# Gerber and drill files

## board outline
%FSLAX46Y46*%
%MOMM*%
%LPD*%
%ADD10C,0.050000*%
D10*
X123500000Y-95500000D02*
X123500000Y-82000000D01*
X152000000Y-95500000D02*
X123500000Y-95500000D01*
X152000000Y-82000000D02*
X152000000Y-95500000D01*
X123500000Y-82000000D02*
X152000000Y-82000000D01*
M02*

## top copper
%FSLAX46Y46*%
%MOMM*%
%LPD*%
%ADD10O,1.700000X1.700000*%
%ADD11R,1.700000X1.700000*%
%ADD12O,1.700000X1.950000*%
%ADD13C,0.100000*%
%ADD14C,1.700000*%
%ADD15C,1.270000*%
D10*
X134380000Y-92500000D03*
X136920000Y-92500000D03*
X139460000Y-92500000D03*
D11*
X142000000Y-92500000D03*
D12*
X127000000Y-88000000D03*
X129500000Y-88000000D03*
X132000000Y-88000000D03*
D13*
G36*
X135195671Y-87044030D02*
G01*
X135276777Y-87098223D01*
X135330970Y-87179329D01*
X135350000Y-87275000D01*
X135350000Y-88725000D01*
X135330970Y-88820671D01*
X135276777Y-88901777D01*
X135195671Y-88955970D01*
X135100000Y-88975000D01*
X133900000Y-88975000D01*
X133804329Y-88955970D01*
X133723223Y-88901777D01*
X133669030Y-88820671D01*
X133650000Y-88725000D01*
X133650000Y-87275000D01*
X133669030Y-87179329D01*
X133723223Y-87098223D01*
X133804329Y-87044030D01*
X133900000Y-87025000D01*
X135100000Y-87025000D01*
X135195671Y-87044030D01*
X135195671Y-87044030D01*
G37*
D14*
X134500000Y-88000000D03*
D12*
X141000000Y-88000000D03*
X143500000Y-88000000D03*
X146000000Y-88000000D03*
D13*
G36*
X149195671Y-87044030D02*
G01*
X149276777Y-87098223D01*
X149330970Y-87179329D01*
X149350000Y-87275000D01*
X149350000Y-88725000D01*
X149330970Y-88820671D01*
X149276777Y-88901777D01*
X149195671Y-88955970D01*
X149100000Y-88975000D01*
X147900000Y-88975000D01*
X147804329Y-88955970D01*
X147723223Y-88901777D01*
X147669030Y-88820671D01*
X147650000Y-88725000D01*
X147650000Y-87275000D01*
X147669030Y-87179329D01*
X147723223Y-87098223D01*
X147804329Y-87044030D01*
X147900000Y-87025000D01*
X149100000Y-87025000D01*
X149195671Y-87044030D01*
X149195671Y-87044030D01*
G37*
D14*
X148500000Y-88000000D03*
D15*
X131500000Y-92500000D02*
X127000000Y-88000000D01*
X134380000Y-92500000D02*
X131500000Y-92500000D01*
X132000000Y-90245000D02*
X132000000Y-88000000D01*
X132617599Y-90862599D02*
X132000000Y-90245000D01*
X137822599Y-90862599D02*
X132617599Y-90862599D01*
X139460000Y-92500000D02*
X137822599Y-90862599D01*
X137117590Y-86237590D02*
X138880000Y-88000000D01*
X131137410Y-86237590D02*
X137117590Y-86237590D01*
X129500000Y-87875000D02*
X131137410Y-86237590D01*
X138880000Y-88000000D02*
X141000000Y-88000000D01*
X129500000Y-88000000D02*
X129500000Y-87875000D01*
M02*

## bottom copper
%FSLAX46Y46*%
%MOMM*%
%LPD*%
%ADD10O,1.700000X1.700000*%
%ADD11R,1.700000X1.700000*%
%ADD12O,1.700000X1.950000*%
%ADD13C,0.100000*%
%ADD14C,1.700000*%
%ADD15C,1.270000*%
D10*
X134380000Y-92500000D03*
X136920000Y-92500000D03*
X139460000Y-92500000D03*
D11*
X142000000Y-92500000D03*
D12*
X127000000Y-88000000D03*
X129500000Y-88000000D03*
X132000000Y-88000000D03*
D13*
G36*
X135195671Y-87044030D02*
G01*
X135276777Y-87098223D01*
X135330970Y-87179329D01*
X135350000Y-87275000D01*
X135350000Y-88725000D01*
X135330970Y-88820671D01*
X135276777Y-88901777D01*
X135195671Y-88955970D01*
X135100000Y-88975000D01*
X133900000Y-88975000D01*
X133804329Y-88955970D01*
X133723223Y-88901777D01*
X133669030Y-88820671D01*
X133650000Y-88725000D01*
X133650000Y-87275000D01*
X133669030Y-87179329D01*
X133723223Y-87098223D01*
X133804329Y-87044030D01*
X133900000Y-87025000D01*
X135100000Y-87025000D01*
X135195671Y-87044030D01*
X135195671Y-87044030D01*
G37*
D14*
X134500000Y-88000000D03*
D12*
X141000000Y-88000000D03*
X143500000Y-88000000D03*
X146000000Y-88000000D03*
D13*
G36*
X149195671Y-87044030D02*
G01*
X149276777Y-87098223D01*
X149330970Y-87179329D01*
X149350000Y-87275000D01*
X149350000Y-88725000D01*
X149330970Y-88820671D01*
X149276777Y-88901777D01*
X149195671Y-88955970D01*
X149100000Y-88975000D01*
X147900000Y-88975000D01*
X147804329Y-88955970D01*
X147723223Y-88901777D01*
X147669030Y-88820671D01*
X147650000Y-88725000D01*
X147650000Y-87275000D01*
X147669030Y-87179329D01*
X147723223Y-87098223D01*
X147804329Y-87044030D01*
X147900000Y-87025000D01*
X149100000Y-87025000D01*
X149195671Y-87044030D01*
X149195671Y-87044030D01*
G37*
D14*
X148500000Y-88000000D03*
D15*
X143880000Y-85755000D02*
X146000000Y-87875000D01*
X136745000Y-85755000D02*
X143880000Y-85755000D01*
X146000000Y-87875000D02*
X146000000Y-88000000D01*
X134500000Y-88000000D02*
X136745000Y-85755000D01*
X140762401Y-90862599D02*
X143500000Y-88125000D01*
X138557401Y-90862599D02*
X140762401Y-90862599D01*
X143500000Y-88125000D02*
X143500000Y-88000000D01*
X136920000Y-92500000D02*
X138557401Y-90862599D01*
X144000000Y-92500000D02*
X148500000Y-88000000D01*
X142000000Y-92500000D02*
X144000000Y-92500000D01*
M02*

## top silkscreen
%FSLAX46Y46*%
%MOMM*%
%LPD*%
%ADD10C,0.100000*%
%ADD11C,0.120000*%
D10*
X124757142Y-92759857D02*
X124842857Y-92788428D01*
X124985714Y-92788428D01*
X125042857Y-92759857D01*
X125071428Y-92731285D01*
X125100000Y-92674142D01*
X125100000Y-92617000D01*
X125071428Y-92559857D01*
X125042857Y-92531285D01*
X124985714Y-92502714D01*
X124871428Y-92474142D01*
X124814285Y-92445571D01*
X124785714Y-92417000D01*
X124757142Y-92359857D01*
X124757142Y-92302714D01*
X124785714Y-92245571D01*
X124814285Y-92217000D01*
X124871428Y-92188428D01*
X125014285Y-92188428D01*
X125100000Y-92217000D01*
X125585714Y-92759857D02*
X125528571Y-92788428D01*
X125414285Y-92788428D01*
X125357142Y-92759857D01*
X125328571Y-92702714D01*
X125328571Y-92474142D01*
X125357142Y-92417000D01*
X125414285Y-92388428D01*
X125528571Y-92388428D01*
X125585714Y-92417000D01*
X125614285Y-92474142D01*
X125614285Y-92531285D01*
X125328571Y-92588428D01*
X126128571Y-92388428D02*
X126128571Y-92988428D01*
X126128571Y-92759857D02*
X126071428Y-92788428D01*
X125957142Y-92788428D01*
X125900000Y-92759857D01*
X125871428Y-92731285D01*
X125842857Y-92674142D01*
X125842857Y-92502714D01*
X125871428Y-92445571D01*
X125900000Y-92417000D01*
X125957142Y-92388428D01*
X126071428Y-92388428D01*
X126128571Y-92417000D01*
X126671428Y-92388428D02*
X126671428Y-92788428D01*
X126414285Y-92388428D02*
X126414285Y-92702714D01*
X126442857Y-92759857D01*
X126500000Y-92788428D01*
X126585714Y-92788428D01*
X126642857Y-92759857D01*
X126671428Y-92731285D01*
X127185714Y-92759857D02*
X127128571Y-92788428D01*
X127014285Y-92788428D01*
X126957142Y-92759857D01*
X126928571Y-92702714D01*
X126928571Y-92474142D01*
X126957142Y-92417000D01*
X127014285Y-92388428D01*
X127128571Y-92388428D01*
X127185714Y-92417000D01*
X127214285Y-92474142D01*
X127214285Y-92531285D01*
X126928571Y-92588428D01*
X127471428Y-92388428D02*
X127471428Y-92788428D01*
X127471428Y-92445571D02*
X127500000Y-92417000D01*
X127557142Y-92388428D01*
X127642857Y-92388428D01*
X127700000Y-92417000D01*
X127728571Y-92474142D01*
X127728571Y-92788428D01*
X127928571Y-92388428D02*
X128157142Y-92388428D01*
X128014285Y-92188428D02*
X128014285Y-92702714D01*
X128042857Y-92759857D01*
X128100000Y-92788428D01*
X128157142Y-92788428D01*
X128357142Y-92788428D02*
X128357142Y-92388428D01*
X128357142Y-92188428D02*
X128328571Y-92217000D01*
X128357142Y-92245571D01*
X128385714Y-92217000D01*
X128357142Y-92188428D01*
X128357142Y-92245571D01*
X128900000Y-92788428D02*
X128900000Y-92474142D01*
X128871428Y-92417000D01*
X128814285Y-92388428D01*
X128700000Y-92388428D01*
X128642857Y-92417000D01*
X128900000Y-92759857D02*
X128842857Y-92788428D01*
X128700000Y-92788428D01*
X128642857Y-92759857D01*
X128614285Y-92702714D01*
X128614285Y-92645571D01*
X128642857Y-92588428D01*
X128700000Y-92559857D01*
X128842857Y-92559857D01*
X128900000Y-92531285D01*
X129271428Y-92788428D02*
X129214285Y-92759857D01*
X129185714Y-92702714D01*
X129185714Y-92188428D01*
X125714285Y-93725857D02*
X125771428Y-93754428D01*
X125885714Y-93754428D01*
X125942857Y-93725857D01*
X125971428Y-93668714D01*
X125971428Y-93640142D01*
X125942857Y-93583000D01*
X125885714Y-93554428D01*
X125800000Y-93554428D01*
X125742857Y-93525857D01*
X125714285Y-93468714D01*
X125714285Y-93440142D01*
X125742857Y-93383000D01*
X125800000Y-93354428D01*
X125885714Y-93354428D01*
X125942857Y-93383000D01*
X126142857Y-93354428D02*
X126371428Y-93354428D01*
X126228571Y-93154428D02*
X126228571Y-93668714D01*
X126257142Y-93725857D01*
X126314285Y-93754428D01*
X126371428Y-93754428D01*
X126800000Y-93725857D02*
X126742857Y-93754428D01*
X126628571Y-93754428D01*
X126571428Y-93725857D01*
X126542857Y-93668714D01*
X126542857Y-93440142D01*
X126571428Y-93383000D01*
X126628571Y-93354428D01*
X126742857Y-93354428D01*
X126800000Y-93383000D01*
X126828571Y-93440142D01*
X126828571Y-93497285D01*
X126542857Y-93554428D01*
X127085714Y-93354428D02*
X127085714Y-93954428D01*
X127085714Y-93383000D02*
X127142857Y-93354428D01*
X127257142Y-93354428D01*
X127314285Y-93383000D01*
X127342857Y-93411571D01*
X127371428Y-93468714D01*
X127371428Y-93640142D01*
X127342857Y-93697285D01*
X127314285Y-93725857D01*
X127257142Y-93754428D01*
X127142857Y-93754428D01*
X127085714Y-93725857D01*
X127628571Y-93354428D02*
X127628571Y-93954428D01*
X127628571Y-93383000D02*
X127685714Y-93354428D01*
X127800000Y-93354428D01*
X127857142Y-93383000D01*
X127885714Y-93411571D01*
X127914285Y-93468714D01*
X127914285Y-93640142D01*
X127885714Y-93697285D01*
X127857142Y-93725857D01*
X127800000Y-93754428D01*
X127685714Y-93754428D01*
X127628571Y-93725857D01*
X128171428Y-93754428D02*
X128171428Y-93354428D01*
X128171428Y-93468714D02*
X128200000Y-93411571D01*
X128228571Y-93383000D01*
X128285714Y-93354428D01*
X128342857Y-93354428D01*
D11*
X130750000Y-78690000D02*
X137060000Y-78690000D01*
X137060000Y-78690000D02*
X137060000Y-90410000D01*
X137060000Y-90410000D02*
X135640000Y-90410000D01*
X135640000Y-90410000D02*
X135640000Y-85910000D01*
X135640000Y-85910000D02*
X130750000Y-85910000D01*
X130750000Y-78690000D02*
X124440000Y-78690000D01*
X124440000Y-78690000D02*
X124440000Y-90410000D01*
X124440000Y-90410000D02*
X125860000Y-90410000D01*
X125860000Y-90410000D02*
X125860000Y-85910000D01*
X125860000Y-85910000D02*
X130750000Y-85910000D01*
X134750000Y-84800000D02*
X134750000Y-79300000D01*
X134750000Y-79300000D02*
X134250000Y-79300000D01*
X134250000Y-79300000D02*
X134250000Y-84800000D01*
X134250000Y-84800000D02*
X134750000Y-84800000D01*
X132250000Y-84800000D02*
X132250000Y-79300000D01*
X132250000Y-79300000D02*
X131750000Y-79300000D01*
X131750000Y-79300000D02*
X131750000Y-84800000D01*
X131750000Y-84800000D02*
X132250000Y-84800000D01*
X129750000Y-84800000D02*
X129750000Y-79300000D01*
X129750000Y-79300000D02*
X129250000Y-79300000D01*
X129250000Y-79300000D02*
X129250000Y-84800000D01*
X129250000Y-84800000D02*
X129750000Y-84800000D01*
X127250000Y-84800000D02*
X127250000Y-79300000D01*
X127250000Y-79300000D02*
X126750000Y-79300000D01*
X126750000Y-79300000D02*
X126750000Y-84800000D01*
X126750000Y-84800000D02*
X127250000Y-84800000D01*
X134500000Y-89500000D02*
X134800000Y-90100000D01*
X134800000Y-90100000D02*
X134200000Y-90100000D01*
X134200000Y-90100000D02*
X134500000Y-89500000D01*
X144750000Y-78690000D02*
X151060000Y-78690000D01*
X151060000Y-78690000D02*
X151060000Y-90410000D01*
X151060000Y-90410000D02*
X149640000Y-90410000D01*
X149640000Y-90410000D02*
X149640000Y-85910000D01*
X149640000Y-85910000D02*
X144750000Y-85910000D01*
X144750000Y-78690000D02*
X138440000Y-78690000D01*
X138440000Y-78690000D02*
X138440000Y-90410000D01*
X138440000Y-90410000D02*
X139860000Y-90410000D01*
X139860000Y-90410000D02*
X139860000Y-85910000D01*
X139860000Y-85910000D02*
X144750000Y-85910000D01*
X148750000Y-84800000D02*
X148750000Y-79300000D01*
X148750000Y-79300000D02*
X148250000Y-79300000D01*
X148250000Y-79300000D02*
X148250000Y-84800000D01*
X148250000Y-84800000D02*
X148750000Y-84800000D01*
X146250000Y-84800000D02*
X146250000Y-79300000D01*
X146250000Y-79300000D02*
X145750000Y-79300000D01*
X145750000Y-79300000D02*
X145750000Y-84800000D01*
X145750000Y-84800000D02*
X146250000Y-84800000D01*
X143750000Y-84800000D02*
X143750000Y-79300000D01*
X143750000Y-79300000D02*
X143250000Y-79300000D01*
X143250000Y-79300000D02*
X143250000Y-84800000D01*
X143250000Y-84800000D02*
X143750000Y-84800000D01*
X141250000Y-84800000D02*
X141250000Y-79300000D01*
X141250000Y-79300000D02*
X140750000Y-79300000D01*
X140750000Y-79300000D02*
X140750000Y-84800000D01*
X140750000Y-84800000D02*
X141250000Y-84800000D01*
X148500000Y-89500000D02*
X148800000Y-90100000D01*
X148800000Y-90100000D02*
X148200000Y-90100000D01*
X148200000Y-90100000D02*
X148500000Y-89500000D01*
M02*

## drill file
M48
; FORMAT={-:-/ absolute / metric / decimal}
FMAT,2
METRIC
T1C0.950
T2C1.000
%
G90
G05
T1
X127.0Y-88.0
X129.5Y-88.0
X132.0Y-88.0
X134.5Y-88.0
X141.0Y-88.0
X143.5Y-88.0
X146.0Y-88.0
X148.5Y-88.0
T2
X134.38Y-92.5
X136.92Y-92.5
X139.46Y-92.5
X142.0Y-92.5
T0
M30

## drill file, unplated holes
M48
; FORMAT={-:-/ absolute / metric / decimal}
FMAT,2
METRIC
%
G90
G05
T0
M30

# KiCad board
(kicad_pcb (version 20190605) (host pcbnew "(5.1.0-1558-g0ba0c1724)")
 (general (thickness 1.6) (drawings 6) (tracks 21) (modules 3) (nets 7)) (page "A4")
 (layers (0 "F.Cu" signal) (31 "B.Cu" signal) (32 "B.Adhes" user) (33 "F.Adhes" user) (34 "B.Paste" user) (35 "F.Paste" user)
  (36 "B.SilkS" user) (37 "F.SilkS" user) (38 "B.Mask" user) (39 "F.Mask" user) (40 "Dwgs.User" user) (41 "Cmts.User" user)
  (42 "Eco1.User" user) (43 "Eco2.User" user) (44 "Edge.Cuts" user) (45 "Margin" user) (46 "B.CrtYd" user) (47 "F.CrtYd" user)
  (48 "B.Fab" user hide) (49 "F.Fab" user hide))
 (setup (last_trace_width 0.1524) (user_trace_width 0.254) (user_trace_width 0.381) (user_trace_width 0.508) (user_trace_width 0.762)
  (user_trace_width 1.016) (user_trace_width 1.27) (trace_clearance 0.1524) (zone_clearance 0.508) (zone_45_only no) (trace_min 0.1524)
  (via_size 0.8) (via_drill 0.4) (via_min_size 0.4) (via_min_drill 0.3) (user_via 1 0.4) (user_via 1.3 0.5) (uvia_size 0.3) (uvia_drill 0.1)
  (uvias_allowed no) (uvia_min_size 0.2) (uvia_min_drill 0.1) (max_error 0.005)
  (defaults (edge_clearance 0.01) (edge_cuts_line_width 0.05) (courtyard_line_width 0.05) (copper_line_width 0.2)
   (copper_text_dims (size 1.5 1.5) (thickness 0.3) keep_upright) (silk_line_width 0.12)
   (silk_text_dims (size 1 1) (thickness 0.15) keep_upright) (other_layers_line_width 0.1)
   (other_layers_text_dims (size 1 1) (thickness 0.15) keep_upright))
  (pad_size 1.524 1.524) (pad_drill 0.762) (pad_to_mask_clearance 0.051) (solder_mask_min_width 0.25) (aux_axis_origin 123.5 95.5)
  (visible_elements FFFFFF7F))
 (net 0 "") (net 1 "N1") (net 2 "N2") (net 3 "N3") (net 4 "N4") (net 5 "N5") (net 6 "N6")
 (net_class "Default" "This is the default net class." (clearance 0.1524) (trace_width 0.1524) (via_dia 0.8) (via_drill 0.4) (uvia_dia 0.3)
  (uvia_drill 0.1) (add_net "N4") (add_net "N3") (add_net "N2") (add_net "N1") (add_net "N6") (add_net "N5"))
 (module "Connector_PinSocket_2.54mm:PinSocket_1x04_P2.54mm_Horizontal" (layer "B.Cu") (at 142 92.5 90)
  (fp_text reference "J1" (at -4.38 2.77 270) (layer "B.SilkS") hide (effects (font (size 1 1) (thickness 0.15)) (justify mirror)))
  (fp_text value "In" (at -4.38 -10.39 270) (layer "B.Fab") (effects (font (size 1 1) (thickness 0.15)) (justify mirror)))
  (pad "4" thru_hole oval (at 0 -7.62 90) (size 1.7 1.7) (drill 1) (layers *.Cu *.Mask) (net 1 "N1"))
  (pad "3" thru_hole oval (at 0 -5.08 90) (size 1.7 1.7) (drill 1) (layers *.Cu *.Mask) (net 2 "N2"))
  (pad "2" thru_hole oval (at 0 -2.54 90) (size 1.7 1.7) (drill 1) (layers *.Cu *.Mask) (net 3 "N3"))
  (pad "1" thru_hole rect (at 0 0 90) (size 1.7 1.7) (drill 1) (layers *.Cu *.Mask) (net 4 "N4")))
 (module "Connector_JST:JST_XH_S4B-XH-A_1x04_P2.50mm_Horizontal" (layer "F.Cu") (at 134.5 88 180)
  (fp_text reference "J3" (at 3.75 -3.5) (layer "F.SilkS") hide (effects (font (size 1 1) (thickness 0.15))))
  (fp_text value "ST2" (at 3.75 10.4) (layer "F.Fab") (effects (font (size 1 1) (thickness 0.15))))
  (fp_line (start 3.75 9.31) (end -2.56 9.31) (layer "F.SilkS") (width 0.12))
  (fp_line (start -2.56 9.31) (end -2.56 -2.41) (layer "F.SilkS") (width 0.12))
  (fp_line (start -2.56 -2.41) (end -1.14 -2.41) (layer "F.SilkS") (width 0.12))
  (fp_line (start -1.14 -2.41) (end -1.14 2.09) (layer "F.SilkS") (width 0.12))
  (fp_line (start -1.14 2.09) (end 3.75 2.09) (layer "F.SilkS") (width 0.12))
  (fp_line (start 3.75 9.31) (end 10.06 9.31) (layer "F.SilkS") (width 0.12))
  (fp_line (start 10.06 9.31) (end 10.06 -2.41) (layer "F.SilkS") (width 0.12))
  (fp_line (start 10.06 -2.41) (end 8.64 -2.41) (layer "F.SilkS") (width 0.12))
  (fp_line (start 8.64 -2.41) (end 8.64 2.09) (layer "F.SilkS") (width 0.12))
  (fp_line (start 8.64 2.09) (end 3.75 2.09) (layer "F.SilkS") (width 0.12))
  (fp_line (start -0.25 3.2) (end -0.25 8.7) (layer "F.SilkS") (width 0.12))
  (fp_line (start -0.25 8.7) (end 0.25 8.7) (layer "F.SilkS") (width 0.12))
  (fp_line (start 0.25 8.7) (end 0.25 3.2) (layer "F.SilkS") (width 0.12))
  (fp_line (start 0.25 3.2) (end -0.25 3.2) (layer "F.SilkS") (width 0.12))
  (fp_line (start 2.25 3.2) (end 2.25 8.7) (layer "F.SilkS") (width 0.12))
  (fp_line (start 2.25 8.7) (end 2.75 8.7) (layer "F.SilkS") (width 0.12))
  (fp_line (start 2.75 8.7) (end 2.75 3.2) (layer "F.SilkS") (width 0.12))
  (fp_line (start 2.75 3.2) (end 2.25 3.2) (layer "F.SilkS") (width 0.12))
  (fp_line (start 4.75 3.2) (end 4.75 8.7) (layer "F.SilkS") (width 0.12))
  (fp_line (start 4.75 8.7) (end 5.25 8.7) (layer "F.SilkS") (width 0.12))
  (fp_line (start 5.25 8.7) (end 5.25 3.2) (layer "F.SilkS") (width 0.12))
  (fp_line (start 5.25 3.2) (end 4.75 3.2) (layer "F.SilkS") (width 0.12))
  (fp_line (start 7.25 3.2) (end 7.25 8.7) (layer "F.SilkS") (width 0.12))
  (fp_line (start 7.25 8.7) (end 7.75 8.7) (layer "F.SilkS") (width 0.12))
  (fp_line (start 7.75 8.7) (end 7.75 3.2) (layer "F.SilkS") (width 0.12))
  (fp_line (start 7.75 3.2) (end 7.25 3.2) (layer "F.SilkS") (width 0.12))
  (fp_line (start 0 -1.5) (end -0.3 -2.1) (layer "F.SilkS") (width 0.12))
  (fp_line (start -0.3 -2.1) (end 0.3 -2.1) (layer "F.SilkS") (width 0.12))
  (fp_line (start 0.3 -2.1) (end 0 -1.5) (layer "F.SilkS") (width 0.12))
  (pad "4" thru_hole oval (at 7.5 0 180) (size 1.7 1.95) (drill 0.95) (layers *.Cu *.Mask) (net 1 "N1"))
  (pad "3" thru_hole oval (at 5 0 180) (size 1.7 1.95) (drill 0.95) (layers *.Cu *.Mask) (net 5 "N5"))
  (pad "2" thru_hole oval (at 2.5 0 180) (size 1.7 1.95) (drill 0.95) (layers *.Cu *.Mask) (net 3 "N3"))
  (pad "1" thru_hole roundrect (at 0 0 180) (size 1.7 1.95) (drill 0.95) (layers *.Cu *.Mask) (roundrect_rratio 0.147059) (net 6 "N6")))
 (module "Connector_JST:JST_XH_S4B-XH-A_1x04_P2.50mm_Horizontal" (layer "F.Cu") (at 148.5 88 180)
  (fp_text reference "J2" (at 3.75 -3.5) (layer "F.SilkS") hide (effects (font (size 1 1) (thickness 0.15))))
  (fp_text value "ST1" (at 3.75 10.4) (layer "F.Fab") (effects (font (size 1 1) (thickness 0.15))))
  (fp_line (start 3.75 9.31) (end -2.56 9.31) (layer "F.SilkS") (width 0.12))
  (fp_line (start -2.56 9.31) (end -2.56 -2.41) (layer "F.SilkS") (width 0.12))
  (fp_line (start -2.56 -2.41) (end -1.14 -2.41) (layer "F.SilkS") (width 0.12))
  (fp_line (start -1.14 -2.41) (end -1.14 2.09) (layer "F.SilkS") (width 0.12))
  (fp_line (start -1.14 2.09) (end 3.75 2.09) (layer "F.SilkS") (width 0.12))
  (fp_line (start 3.75 9.31) (end 10.06 9.31) (layer "F.SilkS") (width 0.12))
  (fp_line (start 10.06 9.31) (end 10.06 -2.41) (layer "F.SilkS") (width 0.12))
  (fp_line (start 10.06 -2.41) (end 8.64 -2.41) (layer "F.SilkS") (width 0.12))
  (fp_line (start 8.64 -2.41) (end 8.64 2.09) (layer "F.SilkS") (width 0.12))
  (fp_line (start 8.64 2.09) (end 3.75 2.09) (layer "F.SilkS") (width 0.12))
  (fp_line (start -0.25 3.2) (end -0.25 8.7) (layer "F.SilkS") (width 0.12))
  (fp_line (start -0.25 8.7) (end 0.25 8.7) (layer "F.SilkS") (width 0.12))
  (fp_line (start 0.25 8.7) (end 0.25 3.2) (layer "F.SilkS") (width 0.12))
  (fp_line (start 0.25 3.2) (end -0.25 3.2) (layer "F.SilkS") (width 0.12))
  (fp_line (start 2.25 3.2) (end 2.25 8.7) (layer "F.SilkS") (width 0.12))
  (fp_line (start 2.25 8.7) (end 2.75 8.7) (layer "F.SilkS") (width 0.12))
  (fp_line (start 2.75 8.7) (end 2.75 3.2) (layer "F.SilkS") (width 0.12))
  (fp_line (start 2.75 3.2) (end 2.25 3.2) (layer "F.SilkS") (width 0.12))
  (fp_line (start 4.75 3.2) (end 4.75 8.7) (layer "F.SilkS") (width 0.12))
  (fp_line (start 4.75 8.7) (end 5.25 8.7) (layer "F.SilkS") (width 0.12))
  (fp_line (start 5.25 8.7) (end 5.25 3.2) (layer "F.SilkS") (width 0.12))
  (fp_line (start 5.25 3.2) (end 4.75 3.2) (layer "F.SilkS") (width 0.12))
  (fp_line (start 7.25 3.2) (end 7.25 8.7) (layer "F.SilkS") (width 0.12))
  (fp_line (start 7.25 8.7) (end 7.75 8.7) (layer "F.SilkS") (width 0.12))
  (fp_line (start 7.75 8.7) (end 7.75 3.2) (layer "F.SilkS") (width 0.12))
  (fp_line (start 7.75 3.2) (end 7.25 3.2) (layer "F.SilkS") (width 0.12))
  (fp_line (start 0 -1.5) (end -0.3 -2.1) (layer "F.SilkS") (width 0.12))
  (fp_line (start -0.3 -2.1) (end 0.3 -2.1) (layer "F.SilkS") (width 0.12))
  (fp_line (start 0.3 -2.1) (end 0 -1.5) (layer "F.SilkS") (width 0.12))
  (pad "4" thru_hole oval (at 7.5 0 180) (size 1.7 1.95) (drill 0.95) (layers *.Cu *.Mask) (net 5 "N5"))
  (pad "3" thru_hole oval (at 5 0 180) (size 1.7 1.95) (drill 0.95) (layers *.Cu *.Mask) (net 2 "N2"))
  (pad "2" thru_hole oval (at 2.5 0 180) (size 1.7 1.95) (drill 0.95) (layers *.Cu *.Mask) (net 6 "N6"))
  (pad "1" thru_hole roundrect (at 0 0 180) (size 1.7 1.95) (drill 0.95) (layers *.Cu *.Mask) (roundrect_rratio 0.147059) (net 4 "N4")))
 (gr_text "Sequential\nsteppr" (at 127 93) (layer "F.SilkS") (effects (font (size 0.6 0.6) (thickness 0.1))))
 (gr_line (start 123.5 95.5) (end 123.5 82) (layer "Edge.Cuts") (width 0.05))
 (gr_line (start 152 95.5) (end 123.5 95.5) (layer "Edge.Cuts") (width 0.05))
 (gr_line (start 152 82) (end 152 95.5) (layer "Edge.Cuts") (width 0.05))
 (gr_line (start 123.5 82) (end 152 82) (layer "Edge.Cuts") (width 0.05))
 (segment (start 131.5 92.5) (end 127 88) (width 1.27) (layer "F.Cu") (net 1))
 (segment (start 134.38 92.5) (end 131.5 92.5) (width 1.27) (layer "F.Cu") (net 1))
 (segment (start 132 90.245) (end 132 88) (width 1.27) (layer "F.Cu") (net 3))
 (segment (start 132.617599 90.862599) (end 132 90.245) (width 1.27) (layer "F.Cu") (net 3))
 (segment (start 137.822599 90.862599) (end 132.617599 90.862599) (width 1.27) (layer "F.Cu") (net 3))
 (segment (start 139.46 92.5) (end 137.822599 90.862599) (width 1.27) (layer "F.Cu") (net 3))
 (segment (start 137.11759 86.23759) (end 138.88 88) (width 1.27) (layer "F.Cu") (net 5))
 (segment (start 131.13741 86.23759) (end 137.11759 86.23759) (width 1.27) (layer "F.Cu") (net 5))
 (segment (start 129.5 87.875) (end 131.13741 86.23759) (width 1.27) (layer "F.Cu") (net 5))
 (segment (start 138.88 88) (end 141 88) (width 1.27) (layer "F.Cu") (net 5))
 (segment (start 129.5 88) (end 129.5 87.875) (width 1.27) (layer "F.Cu") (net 5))
 (segment (start 143.88 85.755) (end 146 87.875) (width 1.27) (layer "B.Cu") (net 6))
 (segment (start 136.745 85.755) (end 143.88 85.755) (width 1.27) (layer "B.Cu") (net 6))
 (segment (start 146 87.875) (end 146 88) (width 1.27) (layer "B.Cu") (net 6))
 (segment (start 134.5 88) (end 136.745 85.755) (width 1.27) (layer "B.Cu") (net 6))
 (segment (start 140.762401 90.862599) (end 143.5 88.125) (width 1.27) (layer "B.Cu") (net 2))
 (segment (start 138.557401 90.862599) (end 140.762401 90.862599) (width 1.27) (layer "B.Cu") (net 2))
 (segment (start 143.5 88.125) (end 143.5 88) (width 1.27) (layer "B.Cu") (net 2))
 (segment (start 136.92 92.5) (end 138.557401 90.862599) (width 1.27) (layer "B.Cu") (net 2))
 (segment (start 144 92.5) (end 148.5 88) (width 1.27) (layer "B.Cu") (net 4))
 (segment (start 142 92.5) (end 144 92.5) (width 1.27) (layer "B.Cu") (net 4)))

